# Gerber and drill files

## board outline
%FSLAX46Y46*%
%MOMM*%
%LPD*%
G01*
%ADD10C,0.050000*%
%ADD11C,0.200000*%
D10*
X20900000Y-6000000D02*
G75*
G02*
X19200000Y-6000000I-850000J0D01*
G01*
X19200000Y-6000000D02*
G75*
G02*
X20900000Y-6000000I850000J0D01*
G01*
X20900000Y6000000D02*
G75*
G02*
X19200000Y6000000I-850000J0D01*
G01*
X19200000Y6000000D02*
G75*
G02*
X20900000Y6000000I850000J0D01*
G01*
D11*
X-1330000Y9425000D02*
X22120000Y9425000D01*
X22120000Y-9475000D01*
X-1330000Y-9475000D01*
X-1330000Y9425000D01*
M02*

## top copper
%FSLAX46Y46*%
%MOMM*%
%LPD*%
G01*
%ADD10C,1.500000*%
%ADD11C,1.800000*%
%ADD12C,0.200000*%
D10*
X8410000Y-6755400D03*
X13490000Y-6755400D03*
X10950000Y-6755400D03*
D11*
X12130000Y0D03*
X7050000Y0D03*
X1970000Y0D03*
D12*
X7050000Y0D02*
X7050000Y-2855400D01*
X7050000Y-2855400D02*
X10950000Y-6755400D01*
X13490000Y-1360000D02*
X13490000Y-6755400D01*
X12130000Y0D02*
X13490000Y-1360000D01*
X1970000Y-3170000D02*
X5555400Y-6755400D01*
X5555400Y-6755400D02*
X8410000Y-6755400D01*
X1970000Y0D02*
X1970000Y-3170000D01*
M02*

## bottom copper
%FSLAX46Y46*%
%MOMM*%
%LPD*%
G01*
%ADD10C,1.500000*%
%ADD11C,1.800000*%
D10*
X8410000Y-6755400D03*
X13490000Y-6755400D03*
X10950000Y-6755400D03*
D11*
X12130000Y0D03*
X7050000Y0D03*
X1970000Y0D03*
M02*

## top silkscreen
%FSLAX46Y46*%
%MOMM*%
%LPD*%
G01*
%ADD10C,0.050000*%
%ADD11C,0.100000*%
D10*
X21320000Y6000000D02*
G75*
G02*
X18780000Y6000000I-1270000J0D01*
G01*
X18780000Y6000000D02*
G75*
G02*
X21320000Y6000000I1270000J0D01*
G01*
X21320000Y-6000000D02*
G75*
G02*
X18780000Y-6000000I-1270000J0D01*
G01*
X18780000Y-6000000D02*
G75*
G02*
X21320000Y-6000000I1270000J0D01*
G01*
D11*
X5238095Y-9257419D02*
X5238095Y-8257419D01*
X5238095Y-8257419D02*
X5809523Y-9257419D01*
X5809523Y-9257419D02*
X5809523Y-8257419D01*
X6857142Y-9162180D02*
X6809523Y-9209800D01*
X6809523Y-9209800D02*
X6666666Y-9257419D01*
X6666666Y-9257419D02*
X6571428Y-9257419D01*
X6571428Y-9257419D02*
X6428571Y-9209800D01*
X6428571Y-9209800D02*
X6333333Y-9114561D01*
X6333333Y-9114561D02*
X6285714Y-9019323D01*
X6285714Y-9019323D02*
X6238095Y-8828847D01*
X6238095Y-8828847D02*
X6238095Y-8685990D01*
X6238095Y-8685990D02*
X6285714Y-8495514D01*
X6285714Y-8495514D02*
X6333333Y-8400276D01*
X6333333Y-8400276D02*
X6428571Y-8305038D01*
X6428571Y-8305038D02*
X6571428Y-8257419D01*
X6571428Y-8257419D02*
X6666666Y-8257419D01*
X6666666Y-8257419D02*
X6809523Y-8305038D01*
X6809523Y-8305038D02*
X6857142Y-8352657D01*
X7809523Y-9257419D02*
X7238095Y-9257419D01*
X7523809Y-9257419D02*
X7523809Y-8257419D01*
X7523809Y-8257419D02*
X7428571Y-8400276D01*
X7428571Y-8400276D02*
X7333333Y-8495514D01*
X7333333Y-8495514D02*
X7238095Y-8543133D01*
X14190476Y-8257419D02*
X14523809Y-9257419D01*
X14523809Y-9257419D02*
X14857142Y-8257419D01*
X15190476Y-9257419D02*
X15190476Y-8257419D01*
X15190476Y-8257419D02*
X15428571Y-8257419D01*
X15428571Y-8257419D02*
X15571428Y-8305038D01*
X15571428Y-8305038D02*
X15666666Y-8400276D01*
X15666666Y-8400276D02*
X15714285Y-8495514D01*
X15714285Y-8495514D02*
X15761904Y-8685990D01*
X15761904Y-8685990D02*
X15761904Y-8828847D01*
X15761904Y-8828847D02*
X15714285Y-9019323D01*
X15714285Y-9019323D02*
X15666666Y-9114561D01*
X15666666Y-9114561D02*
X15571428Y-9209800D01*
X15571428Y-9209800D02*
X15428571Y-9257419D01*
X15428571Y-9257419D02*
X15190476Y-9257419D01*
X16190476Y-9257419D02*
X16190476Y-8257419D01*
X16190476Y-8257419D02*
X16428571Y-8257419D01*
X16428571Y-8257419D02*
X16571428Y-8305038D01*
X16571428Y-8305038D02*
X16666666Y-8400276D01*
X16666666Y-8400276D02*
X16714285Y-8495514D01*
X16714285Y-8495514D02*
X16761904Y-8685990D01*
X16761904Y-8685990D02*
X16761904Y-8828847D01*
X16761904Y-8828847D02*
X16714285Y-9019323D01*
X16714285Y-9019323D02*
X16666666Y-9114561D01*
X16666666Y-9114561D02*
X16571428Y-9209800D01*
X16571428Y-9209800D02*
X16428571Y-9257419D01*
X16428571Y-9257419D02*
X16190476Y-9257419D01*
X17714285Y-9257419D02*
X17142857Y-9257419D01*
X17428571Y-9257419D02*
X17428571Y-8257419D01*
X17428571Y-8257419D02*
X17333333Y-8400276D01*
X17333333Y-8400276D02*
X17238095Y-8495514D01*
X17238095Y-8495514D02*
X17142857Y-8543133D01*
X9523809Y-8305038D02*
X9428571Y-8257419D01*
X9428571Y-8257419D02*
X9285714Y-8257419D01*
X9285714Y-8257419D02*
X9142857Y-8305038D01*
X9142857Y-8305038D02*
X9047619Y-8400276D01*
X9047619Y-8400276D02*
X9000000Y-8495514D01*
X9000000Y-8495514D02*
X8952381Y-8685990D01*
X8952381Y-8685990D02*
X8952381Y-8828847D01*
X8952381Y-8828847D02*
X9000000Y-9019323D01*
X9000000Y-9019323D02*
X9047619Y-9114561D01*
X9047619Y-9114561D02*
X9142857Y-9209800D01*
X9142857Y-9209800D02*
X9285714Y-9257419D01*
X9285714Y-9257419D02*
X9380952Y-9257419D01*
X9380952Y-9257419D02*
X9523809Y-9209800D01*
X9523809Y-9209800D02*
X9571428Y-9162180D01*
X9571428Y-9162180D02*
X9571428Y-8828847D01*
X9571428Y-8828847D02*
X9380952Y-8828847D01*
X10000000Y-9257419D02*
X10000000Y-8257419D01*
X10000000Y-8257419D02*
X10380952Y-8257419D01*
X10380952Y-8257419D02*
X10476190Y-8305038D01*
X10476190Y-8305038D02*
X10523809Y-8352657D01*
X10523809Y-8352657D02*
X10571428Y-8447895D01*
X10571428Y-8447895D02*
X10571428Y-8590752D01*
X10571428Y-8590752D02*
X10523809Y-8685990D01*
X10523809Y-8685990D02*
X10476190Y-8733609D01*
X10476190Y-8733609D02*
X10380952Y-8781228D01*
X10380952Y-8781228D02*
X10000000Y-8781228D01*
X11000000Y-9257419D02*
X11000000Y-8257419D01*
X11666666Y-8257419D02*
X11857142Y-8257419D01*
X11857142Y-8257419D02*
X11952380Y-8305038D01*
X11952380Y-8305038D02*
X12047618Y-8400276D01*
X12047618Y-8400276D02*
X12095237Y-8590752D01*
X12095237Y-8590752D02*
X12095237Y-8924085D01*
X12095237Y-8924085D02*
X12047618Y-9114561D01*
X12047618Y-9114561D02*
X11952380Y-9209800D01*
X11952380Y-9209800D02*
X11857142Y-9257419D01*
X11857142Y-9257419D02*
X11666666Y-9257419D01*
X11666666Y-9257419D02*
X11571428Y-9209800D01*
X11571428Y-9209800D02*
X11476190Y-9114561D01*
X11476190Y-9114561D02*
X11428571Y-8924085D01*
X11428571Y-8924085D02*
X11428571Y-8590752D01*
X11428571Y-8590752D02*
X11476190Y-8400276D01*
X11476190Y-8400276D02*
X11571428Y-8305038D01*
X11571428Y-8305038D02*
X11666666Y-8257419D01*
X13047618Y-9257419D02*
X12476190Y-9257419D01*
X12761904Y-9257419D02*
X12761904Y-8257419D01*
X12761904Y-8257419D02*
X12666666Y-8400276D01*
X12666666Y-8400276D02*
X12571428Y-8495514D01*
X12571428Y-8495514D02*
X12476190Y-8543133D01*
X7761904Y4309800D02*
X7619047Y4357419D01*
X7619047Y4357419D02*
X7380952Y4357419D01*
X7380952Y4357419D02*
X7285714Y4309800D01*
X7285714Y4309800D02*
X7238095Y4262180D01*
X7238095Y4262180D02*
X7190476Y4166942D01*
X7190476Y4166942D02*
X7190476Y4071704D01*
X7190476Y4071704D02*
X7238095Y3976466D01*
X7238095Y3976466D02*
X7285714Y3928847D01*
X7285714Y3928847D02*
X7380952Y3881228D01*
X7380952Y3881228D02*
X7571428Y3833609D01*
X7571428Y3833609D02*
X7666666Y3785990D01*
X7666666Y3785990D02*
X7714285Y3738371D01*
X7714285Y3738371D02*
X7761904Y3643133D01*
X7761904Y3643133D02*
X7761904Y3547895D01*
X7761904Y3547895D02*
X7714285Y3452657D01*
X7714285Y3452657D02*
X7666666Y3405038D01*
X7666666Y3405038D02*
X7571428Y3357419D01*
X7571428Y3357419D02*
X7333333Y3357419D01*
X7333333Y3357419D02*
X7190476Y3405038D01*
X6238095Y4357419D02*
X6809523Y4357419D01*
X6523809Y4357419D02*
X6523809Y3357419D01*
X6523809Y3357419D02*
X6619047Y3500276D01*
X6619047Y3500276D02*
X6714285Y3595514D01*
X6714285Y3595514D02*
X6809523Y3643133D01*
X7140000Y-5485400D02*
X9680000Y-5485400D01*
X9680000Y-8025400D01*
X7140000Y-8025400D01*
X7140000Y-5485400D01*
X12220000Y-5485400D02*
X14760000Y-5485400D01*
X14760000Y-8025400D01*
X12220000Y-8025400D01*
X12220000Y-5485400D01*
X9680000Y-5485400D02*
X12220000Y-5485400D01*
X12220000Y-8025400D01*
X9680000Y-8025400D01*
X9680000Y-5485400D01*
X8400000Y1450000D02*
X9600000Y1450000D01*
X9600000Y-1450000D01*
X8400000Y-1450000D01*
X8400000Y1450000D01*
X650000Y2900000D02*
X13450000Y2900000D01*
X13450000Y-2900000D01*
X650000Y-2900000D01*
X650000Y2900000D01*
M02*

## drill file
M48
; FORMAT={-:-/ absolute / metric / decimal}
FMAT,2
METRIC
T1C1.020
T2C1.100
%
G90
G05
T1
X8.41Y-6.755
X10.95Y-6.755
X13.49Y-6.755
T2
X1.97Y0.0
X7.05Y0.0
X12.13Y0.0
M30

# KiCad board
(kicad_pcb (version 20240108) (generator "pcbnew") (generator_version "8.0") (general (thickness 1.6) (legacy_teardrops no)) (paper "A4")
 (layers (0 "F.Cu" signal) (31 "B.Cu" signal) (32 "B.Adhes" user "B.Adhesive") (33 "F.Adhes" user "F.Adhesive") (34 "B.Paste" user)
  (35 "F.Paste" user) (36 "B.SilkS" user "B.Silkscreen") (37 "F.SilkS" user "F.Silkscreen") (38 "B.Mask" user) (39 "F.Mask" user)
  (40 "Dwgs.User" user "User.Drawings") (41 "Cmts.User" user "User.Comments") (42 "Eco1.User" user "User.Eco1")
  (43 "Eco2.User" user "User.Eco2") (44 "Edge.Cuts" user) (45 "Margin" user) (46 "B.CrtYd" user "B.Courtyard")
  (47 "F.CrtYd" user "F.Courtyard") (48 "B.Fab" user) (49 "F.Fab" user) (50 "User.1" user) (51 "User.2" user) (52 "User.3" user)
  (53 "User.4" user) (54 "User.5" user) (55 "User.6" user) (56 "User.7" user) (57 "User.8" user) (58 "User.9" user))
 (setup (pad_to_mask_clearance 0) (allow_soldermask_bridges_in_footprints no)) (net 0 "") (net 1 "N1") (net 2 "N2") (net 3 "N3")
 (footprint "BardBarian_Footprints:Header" (layer "F.Cu") (at 8.41 6.7554)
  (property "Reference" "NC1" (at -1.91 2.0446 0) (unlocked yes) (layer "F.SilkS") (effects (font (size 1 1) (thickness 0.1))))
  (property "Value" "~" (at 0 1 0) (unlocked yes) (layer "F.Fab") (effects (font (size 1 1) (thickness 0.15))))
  (fp_rect (start -1.27 -1.27) (end 1.27 1.27) (stroke (width 0.1) (type default)) (fill none) (layer "F.SilkS"))
  (pad "1" thru_hole circle (at 0 0) (size 1.5 1.5) (drill 1.02) (layers "*.Cu" "*.Mask") (remove_unused_layers no) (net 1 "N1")))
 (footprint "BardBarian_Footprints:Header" (layer "F.Cu") (at 13.49 6.7554)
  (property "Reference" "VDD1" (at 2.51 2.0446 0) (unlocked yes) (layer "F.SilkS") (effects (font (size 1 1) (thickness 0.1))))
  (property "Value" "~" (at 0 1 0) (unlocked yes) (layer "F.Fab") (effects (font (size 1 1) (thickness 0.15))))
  (fp_rect (start -1.27 -1.27) (end 1.27 1.27) (stroke (width 0.1) (type default)) (fill none) (layer "F.SilkS"))
  (pad "1" thru_hole circle (at 0 0) (size 1.5 1.5) (drill 1.02) (layers "*.Cu" "*.Mask") (remove_unused_layers no) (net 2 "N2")))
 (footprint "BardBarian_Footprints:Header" (layer "F.Cu") (at 10.95 6.7554)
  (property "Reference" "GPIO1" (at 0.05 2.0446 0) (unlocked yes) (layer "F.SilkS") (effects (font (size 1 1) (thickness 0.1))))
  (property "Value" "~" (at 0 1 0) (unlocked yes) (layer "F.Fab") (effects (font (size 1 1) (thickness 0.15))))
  (fp_rect (start -1.27 -1.27) (end 1.27 1.27) (stroke (width 0.1) (type default)) (fill none) (layer "F.SilkS"))
  (pad "1" thru_hole circle (at 0 0) (size 1.5 1.5) (drill 1.02) (layers "*.Cu" "*.Mask") (remove_unused_layers no) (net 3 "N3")))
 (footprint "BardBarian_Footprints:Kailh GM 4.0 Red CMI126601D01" (layer "F.Cu") (at 7.05 0 180)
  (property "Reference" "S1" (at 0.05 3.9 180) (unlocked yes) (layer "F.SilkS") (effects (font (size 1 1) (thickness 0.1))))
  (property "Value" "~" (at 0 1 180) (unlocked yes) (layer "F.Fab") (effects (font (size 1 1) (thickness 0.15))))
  (fp_rect (start -2.55 -1.45) (end -1.35 1.45) (stroke (width 0.1) (type default)) (fill none) (layer "F.SilkS"))
  (fp_rect (start -6.4 -2.9) (end 6.4 2.9) (stroke (width 0.1) (type default)) (fill none) (layer "F.SilkS"))
  (pad "1" thru_hole circle (at -5.08 0 180) (size 1.8 1.8) (drill 1.1) (layers "*.Cu" "*.Mask") (remove_unused_layers no) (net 2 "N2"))
  (pad "2" thru_hole circle (at 0 0 180) (size 1.8 1.8) (drill 1.1) (layers "*.Cu" "*.Mask") (remove_unused_layers no) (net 3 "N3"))
  (pad "3" thru_hole circle (at 5.08 0 180) (size 1.8 1.8) (drill 1.1) (layers "*.Cu" "*.Mask") (remove_unused_layers no) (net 1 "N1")))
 (gr_circle (center 20.05 -6) (end 21.32 -6) (stroke (width 0.05) (type default)) (fill none) (layer "F.SilkS"))
 (gr_circle (center 20.05 6) (end 21.32 6) (stroke (width 0.05) (type default)) (fill none) (layer "F.SilkS"))
 (gr_circle (center 20.05 6) (end 20.9 6) (stroke (width 0.05) (type default)) (fill none) (layer "Edge.Cuts"))
 (gr_circle (center 20.05 -6) (end 20.9 -6) (stroke (width 0.05) (type default)) (fill none) (layer "Edge.Cuts"))
 (gr_rect (start -1.33 9.475) (end 22.12 -9.425) (stroke (width 0.2) (type default)) (fill none) (layer "Edge.Cuts"))
 (segment (start 7.05 0) (end 7.05 2.8554) (width 0.2) (layer "F.Cu") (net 3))
 (segment (start 7.05 2.8554) (end 10.95 6.7554) (width 0.2) (layer "F.Cu") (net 3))
 (segment (start 13.49 1.36) (end 13.49 6.7554) (width 0.2) (layer "F.Cu") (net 2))
 (segment (start 12.13 0) (end 13.49 1.36) (width 0.2) (layer "F.Cu") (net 2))
 (segment (start 1.97 3.17) (end 5.5554 6.7554) (width 0.2) (layer "F.Cu") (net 1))
 (segment (start 5.5554 6.7554) (end 8.41 6.7554) (width 0.2) (layer "F.Cu") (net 1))
 (segment (start 1.97 0) (end 1.97 3.17) (width 0.2) (layer "F.Cu") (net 1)))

